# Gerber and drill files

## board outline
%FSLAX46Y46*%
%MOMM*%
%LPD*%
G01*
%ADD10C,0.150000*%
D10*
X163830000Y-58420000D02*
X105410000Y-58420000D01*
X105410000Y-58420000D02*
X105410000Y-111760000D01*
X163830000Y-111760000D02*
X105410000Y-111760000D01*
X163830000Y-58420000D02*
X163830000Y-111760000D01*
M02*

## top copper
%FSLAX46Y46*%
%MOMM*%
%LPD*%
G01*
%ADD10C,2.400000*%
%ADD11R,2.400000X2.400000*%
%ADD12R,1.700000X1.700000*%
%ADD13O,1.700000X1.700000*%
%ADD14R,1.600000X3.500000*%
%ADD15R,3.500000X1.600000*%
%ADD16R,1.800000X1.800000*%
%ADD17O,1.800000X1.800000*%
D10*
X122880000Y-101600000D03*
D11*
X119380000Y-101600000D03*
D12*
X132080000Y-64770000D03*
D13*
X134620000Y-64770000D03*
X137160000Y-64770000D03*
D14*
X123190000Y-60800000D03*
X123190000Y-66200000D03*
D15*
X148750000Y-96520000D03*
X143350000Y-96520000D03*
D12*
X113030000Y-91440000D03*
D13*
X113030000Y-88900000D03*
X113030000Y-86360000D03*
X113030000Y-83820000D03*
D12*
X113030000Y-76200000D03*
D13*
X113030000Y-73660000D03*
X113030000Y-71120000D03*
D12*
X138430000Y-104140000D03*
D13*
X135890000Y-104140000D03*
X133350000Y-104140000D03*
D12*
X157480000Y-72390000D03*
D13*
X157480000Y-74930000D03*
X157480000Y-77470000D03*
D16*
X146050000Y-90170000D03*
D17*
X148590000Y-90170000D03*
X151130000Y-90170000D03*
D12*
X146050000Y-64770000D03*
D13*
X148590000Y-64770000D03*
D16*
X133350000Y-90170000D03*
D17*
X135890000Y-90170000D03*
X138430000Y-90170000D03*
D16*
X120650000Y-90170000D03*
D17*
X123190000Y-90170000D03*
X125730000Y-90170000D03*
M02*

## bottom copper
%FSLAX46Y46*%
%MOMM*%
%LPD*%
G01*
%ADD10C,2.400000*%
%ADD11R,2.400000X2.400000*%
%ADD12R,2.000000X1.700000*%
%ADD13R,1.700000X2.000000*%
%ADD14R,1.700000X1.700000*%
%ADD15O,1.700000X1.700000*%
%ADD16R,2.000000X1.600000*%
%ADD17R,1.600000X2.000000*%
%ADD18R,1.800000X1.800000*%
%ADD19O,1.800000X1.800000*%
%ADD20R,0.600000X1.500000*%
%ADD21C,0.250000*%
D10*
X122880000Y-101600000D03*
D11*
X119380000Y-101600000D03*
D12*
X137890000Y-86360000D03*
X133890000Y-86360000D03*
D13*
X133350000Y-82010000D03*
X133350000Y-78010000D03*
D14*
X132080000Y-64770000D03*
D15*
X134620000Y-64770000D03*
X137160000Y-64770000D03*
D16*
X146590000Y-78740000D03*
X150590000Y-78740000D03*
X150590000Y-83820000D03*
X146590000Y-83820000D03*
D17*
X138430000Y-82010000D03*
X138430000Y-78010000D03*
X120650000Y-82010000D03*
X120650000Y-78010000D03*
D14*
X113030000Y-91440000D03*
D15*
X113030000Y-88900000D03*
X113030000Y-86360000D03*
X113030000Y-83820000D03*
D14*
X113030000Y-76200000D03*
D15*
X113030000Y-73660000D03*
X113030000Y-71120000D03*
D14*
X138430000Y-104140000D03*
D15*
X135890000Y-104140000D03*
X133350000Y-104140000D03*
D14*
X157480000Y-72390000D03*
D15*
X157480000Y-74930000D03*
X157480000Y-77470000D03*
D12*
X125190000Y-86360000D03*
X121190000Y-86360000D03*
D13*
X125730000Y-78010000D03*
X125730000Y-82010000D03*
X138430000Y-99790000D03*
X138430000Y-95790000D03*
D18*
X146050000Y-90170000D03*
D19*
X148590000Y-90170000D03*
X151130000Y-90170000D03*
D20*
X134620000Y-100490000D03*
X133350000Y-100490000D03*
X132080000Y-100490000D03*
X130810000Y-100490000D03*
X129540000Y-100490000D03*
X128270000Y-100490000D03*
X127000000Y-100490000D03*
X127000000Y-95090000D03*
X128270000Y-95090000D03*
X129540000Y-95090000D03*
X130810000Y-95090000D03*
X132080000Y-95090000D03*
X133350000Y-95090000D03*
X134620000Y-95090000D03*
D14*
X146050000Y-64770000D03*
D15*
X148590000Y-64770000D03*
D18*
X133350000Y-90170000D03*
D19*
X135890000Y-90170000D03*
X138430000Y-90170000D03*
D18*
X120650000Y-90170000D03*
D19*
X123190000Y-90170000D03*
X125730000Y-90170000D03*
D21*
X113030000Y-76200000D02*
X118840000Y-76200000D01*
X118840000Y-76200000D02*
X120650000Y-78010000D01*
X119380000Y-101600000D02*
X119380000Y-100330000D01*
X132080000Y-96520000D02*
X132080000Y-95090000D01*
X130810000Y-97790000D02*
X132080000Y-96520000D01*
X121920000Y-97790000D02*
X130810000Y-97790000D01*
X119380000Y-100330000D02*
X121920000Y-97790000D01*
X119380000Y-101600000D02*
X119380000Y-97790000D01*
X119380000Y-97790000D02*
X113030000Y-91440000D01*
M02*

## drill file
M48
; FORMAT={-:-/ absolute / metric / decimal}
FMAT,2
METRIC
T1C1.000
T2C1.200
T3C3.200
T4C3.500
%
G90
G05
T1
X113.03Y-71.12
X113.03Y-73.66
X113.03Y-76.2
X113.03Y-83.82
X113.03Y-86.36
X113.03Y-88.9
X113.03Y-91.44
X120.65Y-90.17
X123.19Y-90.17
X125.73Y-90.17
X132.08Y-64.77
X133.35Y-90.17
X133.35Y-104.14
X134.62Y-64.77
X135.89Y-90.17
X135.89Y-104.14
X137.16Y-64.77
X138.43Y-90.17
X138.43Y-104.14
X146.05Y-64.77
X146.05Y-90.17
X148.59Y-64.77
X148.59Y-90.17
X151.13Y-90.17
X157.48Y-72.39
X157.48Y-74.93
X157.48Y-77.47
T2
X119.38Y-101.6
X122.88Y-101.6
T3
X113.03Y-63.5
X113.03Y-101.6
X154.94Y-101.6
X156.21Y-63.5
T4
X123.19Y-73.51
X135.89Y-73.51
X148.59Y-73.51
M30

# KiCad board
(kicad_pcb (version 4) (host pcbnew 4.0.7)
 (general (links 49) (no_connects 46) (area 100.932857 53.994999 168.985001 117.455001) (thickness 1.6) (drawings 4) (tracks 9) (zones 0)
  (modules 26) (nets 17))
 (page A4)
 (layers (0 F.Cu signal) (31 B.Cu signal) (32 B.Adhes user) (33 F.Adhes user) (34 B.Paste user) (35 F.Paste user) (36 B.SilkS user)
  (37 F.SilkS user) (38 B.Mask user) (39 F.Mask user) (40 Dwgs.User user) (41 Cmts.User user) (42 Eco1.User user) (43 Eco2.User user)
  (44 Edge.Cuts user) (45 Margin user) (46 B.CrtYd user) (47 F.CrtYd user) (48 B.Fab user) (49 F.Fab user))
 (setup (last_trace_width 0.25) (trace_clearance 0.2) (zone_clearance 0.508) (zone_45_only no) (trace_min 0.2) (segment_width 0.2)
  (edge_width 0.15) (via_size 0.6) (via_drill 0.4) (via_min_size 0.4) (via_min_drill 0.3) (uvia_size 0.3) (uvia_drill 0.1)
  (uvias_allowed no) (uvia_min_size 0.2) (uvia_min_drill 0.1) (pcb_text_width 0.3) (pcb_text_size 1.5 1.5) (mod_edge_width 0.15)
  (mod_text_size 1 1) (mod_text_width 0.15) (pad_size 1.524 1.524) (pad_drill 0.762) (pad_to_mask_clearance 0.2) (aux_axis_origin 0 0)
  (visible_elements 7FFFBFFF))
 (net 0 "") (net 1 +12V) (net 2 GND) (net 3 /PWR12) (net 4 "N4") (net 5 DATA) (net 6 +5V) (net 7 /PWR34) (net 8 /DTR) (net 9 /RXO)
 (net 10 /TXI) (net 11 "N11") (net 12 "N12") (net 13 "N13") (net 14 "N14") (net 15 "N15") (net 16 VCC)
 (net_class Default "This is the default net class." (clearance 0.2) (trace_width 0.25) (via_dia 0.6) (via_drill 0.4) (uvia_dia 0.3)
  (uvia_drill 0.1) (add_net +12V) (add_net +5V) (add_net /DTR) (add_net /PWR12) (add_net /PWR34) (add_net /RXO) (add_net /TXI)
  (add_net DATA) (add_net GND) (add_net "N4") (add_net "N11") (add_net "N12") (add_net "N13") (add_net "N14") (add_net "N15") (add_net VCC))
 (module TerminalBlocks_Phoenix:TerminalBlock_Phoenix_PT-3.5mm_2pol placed (layer F.Cu) (at 119.38 101.6)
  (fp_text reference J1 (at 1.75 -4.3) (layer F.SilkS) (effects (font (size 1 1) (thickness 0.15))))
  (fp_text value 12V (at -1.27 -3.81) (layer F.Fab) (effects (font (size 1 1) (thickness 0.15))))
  (pad 2 thru_hole circle (at 3.5 0) (size 2.4 2.4) (drill 1.2) (layers *.Cu *.Mask) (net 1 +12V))
  (pad 1 thru_hole rect (at 0 0) (size 2.4 2.4) (drill 1.2) (layers *.Cu *.Mask) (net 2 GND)))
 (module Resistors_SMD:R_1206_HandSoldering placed (layer B.Cu) (at 135.89 86.36 180)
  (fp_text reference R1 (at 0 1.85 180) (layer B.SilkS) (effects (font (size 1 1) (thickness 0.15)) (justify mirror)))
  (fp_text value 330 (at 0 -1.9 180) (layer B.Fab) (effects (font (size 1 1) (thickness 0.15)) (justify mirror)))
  (pad 1 smd rect (at -2 0 180) (size 2 1.7) (layers B.Cu B.Paste B.Mask) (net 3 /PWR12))
  (pad 2 smd rect (at 2 0 180) (size 2 1.7) (layers B.Cu B.Paste B.Mask) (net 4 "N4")))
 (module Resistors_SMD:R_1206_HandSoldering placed (layer B.Cu) (at 133.35 80.01 90)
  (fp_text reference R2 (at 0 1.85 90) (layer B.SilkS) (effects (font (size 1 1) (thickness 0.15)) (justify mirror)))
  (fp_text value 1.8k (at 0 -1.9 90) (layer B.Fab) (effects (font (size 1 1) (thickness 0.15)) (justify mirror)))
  (pad 1 smd rect (at -2 0 90) (size 2 1.7) (layers B.Cu B.Paste B.Mask) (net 4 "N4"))
  (pad 2 smd rect (at 2 0 90) (size 2 1.7) (layers B.Cu B.Paste B.Mask) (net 2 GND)))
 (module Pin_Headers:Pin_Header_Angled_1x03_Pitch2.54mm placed (layer F.Cu) (at 132.08 64.77 90)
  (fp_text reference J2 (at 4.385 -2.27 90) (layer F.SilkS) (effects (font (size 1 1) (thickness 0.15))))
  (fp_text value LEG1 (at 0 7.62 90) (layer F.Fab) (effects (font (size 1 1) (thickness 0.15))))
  (pad 1 thru_hole rect (at 0 0 90) (size 1.7 1.7) (drill 1) (layers *.Cu *.Mask) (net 2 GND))
  (pad 2 thru_hole oval (at 0 2.54 90) (size 1.7 1.7) (drill 1) (layers *.Cu *.Mask) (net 3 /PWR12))
  (pad 3 thru_hole oval (at 0 5.08 90) (size 1.7 1.7) (drill 1) (layers *.Cu *.Mask) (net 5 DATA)))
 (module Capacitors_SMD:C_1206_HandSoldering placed (layer B.Cu) (at 148.59 78.74)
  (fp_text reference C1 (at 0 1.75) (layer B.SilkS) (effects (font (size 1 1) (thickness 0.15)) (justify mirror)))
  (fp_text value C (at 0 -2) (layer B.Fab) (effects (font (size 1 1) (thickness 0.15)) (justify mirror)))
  (pad 1 smd rect (at -2 0) (size 2 1.6) (layers B.Cu B.Paste B.Mask) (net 1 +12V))
  (pad 2 smd rect (at 2 0) (size 2 1.6) (layers B.Cu B.Paste B.Mask) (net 2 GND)))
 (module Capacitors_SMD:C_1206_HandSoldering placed (layer B.Cu) (at 148.59 83.82 180)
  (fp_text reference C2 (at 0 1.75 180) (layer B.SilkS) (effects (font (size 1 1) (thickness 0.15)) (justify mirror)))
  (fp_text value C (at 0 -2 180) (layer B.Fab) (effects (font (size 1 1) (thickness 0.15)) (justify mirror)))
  (pad 1 smd rect (at -2 0 180) (size 2 1.6) (layers B.Cu B.Paste B.Mask) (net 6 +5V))
  (pad 2 smd rect (at 2 0 180) (size 2 1.6) (layers B.Cu B.Paste B.Mask) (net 2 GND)))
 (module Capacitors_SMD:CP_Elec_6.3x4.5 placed (layer F.Cu) (at 123.19 63.5 270)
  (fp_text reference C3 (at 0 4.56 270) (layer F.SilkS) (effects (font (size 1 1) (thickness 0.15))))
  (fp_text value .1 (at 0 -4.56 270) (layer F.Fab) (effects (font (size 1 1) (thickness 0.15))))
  (pad 1 smd rect (at -2.7 0 90) (size 3.5 1.6) (layers F.Cu F.Paste F.Mask) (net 3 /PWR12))
  (pad 2 smd rect (at 2.7 0 90) (size 3.5 1.6) (layers F.Cu F.Paste F.Mask) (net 2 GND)))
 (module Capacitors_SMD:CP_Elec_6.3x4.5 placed (layer F.Cu) (at 146.05 96.52 180)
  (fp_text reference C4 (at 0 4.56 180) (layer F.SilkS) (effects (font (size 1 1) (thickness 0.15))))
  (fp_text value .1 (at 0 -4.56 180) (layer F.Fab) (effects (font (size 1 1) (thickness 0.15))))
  (pad 1 smd rect (at -2.7 0) (size 3.5 1.6) (layers F.Cu F.Paste F.Mask) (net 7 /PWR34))
  (pad 2 smd rect (at 2.7 0) (size 3.5 1.6) (layers F.Cu F.Paste F.Mask) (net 2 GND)))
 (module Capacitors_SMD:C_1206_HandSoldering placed (layer B.Cu) (at 138.43 80.01 90)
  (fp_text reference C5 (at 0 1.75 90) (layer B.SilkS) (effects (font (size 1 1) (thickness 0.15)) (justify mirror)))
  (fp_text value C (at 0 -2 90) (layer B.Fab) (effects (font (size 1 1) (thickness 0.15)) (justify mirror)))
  (pad 1 smd rect (at -2 0 90) (size 2 1.6) (layers B.Cu B.Paste B.Mask) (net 1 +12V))
  (pad 2 smd rect (at 2 0 90) (size 2 1.6) (layers B.Cu B.Paste B.Mask) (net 2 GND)))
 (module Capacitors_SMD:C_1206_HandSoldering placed (layer B.Cu) (at 120.65 80.01 90)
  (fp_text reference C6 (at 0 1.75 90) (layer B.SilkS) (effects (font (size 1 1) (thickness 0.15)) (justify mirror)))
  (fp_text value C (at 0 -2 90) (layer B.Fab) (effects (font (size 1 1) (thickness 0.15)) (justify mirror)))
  (pad 1 smd rect (at -2 0 90) (size 2 1.6) (layers B.Cu B.Paste B.Mask) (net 1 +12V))
  (pad 2 smd rect (at 2 0 90) (size 2 1.6) (layers B.Cu B.Paste B.Mask) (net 2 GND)))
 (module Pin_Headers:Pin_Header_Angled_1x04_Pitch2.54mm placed (layer F.Cu) (at 113.03 91.44 180)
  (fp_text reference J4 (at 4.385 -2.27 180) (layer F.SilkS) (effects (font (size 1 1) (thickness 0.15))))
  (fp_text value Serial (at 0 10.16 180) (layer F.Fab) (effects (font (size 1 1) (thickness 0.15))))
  (pad 1 thru_hole rect (at 0 0 180) (size 1.7 1.7) (drill 1) (layers *.Cu *.Mask) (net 2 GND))
  (pad 2 thru_hole oval (at 0 2.54 180) (size 1.7 1.7) (drill 1) (layers *.Cu *.Mask) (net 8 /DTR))
  (pad 3 thru_hole oval (at 0 5.08 180) (size 1.7 1.7) (drill 1) (layers *.Cu *.Mask) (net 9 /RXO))
  (pad 4 thru_hole oval (at 0 7.62 180) (size 1.7 1.7) (drill 1) (layers *.Cu *.Mask) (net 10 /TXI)))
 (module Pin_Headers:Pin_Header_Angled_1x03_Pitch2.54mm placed (layer F.Cu) (at 113.03 76.2 180)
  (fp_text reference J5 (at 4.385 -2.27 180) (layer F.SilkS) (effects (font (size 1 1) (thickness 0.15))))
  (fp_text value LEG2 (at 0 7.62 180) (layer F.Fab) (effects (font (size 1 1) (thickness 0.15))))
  (pad 1 thru_hole rect (at 0 0 180) (size 1.7 1.7) (drill 1) (layers *.Cu *.Mask) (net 2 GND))
  (pad 2 thru_hole oval (at 0 2.54 180) (size 1.7 1.7) (drill 1) (layers *.Cu *.Mask) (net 3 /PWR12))
  (pad 3 thru_hole oval (at 0 5.08 180) (size 1.7 1.7) (drill 1) (layers *.Cu *.Mask) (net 5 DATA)))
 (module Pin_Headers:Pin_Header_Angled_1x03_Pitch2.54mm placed (layer F.Cu) (at 138.43 104.14 270)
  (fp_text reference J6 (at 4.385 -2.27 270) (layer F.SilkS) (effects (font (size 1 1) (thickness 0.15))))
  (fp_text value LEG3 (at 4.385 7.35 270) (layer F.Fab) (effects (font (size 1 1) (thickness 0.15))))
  (pad 1 thru_hole rect (at 0 0 270) (size 1.7 1.7) (drill 1) (layers *.Cu *.Mask) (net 2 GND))
  (pad 2 thru_hole oval (at 0 2.54 270) (size 1.7 1.7) (drill 1) (layers *.Cu *.Mask) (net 7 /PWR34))
  (pad 3 thru_hole oval (at 0 5.08 270) (size 1.7 1.7) (drill 1) (layers *.Cu *.Mask) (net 5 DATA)))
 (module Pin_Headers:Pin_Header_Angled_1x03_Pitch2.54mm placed (layer F.Cu) (at 157.48 72.39)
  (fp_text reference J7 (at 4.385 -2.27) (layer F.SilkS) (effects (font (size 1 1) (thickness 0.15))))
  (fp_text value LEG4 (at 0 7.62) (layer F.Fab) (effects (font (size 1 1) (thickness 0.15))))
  (pad 1 thru_hole rect (at 0 0) (size 1.7 1.7) (drill 1) (layers *.Cu *.Mask) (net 2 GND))
  (pad 2 thru_hole oval (at 0 2.54) (size 1.7 1.7) (drill 1) (layers *.Cu *.Mask) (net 7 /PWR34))
  (pad 3 thru_hole oval (at 0 5.08) (size 1.7 1.7) (drill 1) (layers *.Cu *.Mask) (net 5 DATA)))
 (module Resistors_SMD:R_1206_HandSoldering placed (layer B.Cu) (at 123.19 86.36 180)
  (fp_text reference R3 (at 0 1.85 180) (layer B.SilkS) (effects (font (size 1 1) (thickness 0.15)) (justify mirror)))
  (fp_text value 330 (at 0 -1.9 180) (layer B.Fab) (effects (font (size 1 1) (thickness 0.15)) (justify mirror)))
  (pad 1 smd rect (at -2 0 180) (size 2 1.7) (layers B.Cu B.Paste B.Mask) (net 7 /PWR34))
  (pad 2 smd rect (at 2 0 180) (size 2 1.7) (layers B.Cu B.Paste B.Mask) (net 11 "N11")))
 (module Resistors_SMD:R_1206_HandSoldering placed (layer B.Cu) (at 125.73 80.01 270)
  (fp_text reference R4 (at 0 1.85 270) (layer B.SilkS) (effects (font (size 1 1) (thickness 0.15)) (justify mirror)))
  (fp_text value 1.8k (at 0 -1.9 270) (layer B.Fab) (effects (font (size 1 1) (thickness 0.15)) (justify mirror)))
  (pad 1 smd rect (at -2 0 270) (size 2 1.7) (layers B.Cu B.Paste B.Mask) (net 11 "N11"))
  (pad 2 smd rect (at 2 0 270) (size 2 1.7) (layers B.Cu B.Paste B.Mask) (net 2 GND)))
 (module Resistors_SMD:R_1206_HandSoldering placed (layer B.Cu) (at 138.43 97.79 90)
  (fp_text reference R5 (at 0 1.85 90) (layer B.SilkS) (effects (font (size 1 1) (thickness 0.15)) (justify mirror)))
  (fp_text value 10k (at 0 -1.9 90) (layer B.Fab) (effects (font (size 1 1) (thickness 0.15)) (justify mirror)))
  (pad 1 smd rect (at -2 0 90) (size 2 1.7) (layers B.Cu B.Paste B.Mask) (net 6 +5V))
  (pad 2 smd rect (at 2 0 90) (size 2 1.7) (layers B.Cu B.Paste B.Mask) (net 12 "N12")))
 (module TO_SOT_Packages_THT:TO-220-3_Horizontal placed (layer F.Cu) (at 146.05 90.17)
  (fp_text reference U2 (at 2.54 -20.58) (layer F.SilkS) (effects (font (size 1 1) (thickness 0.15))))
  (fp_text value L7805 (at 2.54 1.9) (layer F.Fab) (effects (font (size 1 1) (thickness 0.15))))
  (pad 0 np_thru_hole oval (at 2.54 -16.66) (size 3.5 3.5) (drill 3.5) (layers *.Cu *.Mask))
  (pad 1 thru_hole rect (at 0 0) (size 1.8 1.8) (drill 1) (layers *.Cu *.Mask) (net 1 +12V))
  (pad 2 thru_hole oval (at 2.54 0) (size 1.8 1.8) (drill 1) (layers *.Cu *.Mask) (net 2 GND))
  (pad 3 thru_hole oval (at 5.08 0) (size 1.8 1.8) (drill 1) (layers *.Cu *.Mask) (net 6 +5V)))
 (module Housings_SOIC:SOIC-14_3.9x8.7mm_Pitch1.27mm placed (layer B.Cu) (at 130.81 97.79 90)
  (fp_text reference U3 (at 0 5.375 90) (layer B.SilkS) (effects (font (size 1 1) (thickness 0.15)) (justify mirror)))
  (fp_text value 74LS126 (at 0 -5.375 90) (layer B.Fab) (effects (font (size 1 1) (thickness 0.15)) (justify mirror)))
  (pad 1 smd rect (at -2.7 3.81 90) (size 1.5 0.6) (layers B.Cu B.Paste B.Mask) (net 8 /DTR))
  (pad 2 smd rect (at -2.7 2.54 90) (size 1.5 0.6) (layers B.Cu B.Paste B.Mask) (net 5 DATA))
  (pad 3 smd rect (at -2.7 1.27 90) (size 1.5 0.6) (layers B.Cu B.Paste B.Mask) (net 9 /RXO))
  (pad 4 smd rect (at -2.7 0 90) (size 1.5 0.6) (layers B.Cu B.Paste B.Mask) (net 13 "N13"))
  (pad 5 smd rect (at -2.7 -1.27 90) (size 1.5 0.6) (layers B.Cu B.Paste B.Mask) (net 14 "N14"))
  (pad 6 smd rect (at -2.7 -2.54 90) (size 1.5 0.6) (layers B.Cu B.Paste B.Mask) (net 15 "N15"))
  (pad 7 smd rect (at -2.7 -3.81 90) (size 1.5 0.6) (layers B.Cu B.Paste B.Mask) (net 2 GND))
  (pad 8 smd rect (at 2.7 -3.81 90) (size 1.5 0.6) (layers B.Cu B.Paste B.Mask) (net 5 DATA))
  (pad 9 smd rect (at 2.7 -2.54 90) (size 1.5 0.6) (layers B.Cu B.Paste B.Mask) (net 10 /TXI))
  (pad 10 smd rect (at 2.7 -1.27 90) (size 1.5 0.6) (layers B.Cu B.Paste B.Mask) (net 12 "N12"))
  (pad 11 smd rect (at 2.7 0 90) (size 1.5 0.6) (layers B.Cu B.Paste B.Mask) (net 12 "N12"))
  (pad 12 smd rect (at 2.7 1.27 90) (size 1.5 0.6) (layers B.Cu B.Paste B.Mask) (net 2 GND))
  (pad 13 smd rect (at 2.7 2.54 90) (size 1.5 0.6) (layers B.Cu B.Paste B.Mask) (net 8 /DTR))
  (pad 14 smd rect (at 2.7 3.81 90) (size 1.5 0.6) (layers B.Cu B.Paste B.Mask) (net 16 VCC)))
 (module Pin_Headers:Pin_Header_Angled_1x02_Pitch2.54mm (layer F.Cu) (at 146.05 64.77 90)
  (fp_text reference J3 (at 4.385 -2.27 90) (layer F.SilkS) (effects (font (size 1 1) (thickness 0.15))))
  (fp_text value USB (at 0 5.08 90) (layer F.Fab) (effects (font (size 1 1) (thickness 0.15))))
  (pad 1 thru_hole rect (at 0 0 90) (size 1.7 1.7) (drill 1) (layers *.Cu *.Mask) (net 2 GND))
  (pad 2 thru_hole oval (at 0 2.54 90) (size 1.7 1.7) (drill 1) (layers *.Cu *.Mask) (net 6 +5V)))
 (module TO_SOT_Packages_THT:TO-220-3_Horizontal (layer F.Cu) (at 133.35 90.17)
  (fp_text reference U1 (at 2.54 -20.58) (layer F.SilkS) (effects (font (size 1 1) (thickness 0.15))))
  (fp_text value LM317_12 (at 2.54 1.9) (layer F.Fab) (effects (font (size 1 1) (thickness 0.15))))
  (pad 0 np_thru_hole oval (at 2.54 -16.66) (size 3.5 3.5) (drill 3.5) (layers *.Cu *.Mask))
  (pad 1 thru_hole rect (at 0 0) (size 1.8 1.8) (drill 1) (layers *.Cu *.Mask) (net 4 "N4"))
  (pad 2 thru_hole oval (at 2.54 0) (size 1.8 1.8) (drill 1) (layers *.Cu *.Mask) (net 1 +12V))
  (pad 3 thru_hole oval (at 5.08 0) (size 1.8 1.8) (drill 1) (layers *.Cu *.Mask) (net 3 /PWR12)))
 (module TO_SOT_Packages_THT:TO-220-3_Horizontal (layer F.Cu) (at 120.65 90.17)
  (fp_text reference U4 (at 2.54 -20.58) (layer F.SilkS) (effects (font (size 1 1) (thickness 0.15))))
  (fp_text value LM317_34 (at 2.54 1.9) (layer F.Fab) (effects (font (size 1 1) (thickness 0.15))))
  (pad 0 np_thru_hole oval (at 2.54 -16.66) (size 3.5 3.5) (drill 3.5) (layers *.Cu *.Mask))
  (pad 1 thru_hole rect (at 0 0) (size 1.8 1.8) (drill 1) (layers *.Cu *.Mask) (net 11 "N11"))
  (pad 2 thru_hole oval (at 2.54 0) (size 1.8 1.8) (drill 1) (layers *.Cu *.Mask) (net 1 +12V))
  (pad 3 thru_hole oval (at 5.08 0) (size 1.8 1.8) (drill 1) (layers *.Cu *.Mask) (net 7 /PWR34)))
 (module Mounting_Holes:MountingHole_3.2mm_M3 (layer F.Cu) (at 156.21 63.5)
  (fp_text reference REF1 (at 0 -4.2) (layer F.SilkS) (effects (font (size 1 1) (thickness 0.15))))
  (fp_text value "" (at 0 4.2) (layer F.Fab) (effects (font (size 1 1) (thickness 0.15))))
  (pad 1 np_thru_hole circle (at 0 0) (size 3.2 3.2) (drill 3.2) (layers *.Cu *.Mask)))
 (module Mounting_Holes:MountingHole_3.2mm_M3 (layer F.Cu) (at 113.03 63.5)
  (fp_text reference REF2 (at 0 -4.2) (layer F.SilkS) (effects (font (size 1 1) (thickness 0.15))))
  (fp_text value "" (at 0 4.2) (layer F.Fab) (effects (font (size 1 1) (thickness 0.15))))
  (pad 1 np_thru_hole circle (at 0 0) (size 3.2 3.2) (drill 3.2) (layers *.Cu *.Mask)))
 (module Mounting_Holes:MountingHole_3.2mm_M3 (layer F.Cu) (at 113.03 101.6)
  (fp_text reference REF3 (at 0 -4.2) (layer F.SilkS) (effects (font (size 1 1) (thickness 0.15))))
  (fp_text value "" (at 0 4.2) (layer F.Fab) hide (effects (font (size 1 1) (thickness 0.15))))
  (pad 1 np_thru_hole circle (at 0 0) (size 3.2 3.2) (drill 3.2) (layers *.Cu *.Mask)))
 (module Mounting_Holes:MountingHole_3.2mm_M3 (layer F.Cu) (at 154.94 101.6)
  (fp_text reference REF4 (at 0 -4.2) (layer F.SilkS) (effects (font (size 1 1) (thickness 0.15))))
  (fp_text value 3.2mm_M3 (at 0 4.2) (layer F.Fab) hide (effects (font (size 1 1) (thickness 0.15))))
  (pad 1 np_thru_hole circle (at 0 0) (size 3.2 3.2) (drill 3.2) (layers *.Cu *.Mask)))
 (gr_line (start 163.83 58.42) (end 105.41 58.42) (angle 90) (layer Edge.Cuts) (width 0.15))
 (gr_line (start 105.41 58.42) (end 105.41 111.76) (angle 90) (layer Edge.Cuts) (width 0.15))
 (gr_line (start 163.83 111.76) (end 105.41 111.76) (angle 90) (layer Edge.Cuts) (width 0.15))
 (gr_line (start 163.83 58.42) (end 163.83 111.76) (angle 90) (layer Edge.Cuts) (width 0.15))
 (segment (start 113.03 76.2) (end 118.84 76.2) (width 0.25) (layer B.Cu) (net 2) (status 400000))
 (segment (start 118.84 76.2) (end 120.65 78.01) (width 0.25) (layer B.Cu) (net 2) (status 800000))
 (segment (start 119.38 101.6) (end 119.38 100.33) (width 0.25) (layer B.Cu) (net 2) (status 400000))
 (segment (start 132.08 96.52) (end 132.08 95.09) (width 0.25) (layer B.Cu) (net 2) (status 800000))
 (segment (start 130.81 97.79) (end 132.08 96.52) (width 0.25) (layer B.Cu) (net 2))
 (segment (start 121.92 97.79) (end 130.81 97.79) (width 0.25) (layer B.Cu) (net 2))
 (segment (start 119.38 100.33) (end 121.92 97.79) (width 0.25) (layer B.Cu) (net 2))
 (segment (start 119.38 101.6) (end 119.38 97.79) (width 0.25) (layer B.Cu) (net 2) (status 400000))
 (segment (start 119.38 97.79) (end 113.03 91.44) (width 0.25) (layer B.Cu) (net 2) (status 800000)))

